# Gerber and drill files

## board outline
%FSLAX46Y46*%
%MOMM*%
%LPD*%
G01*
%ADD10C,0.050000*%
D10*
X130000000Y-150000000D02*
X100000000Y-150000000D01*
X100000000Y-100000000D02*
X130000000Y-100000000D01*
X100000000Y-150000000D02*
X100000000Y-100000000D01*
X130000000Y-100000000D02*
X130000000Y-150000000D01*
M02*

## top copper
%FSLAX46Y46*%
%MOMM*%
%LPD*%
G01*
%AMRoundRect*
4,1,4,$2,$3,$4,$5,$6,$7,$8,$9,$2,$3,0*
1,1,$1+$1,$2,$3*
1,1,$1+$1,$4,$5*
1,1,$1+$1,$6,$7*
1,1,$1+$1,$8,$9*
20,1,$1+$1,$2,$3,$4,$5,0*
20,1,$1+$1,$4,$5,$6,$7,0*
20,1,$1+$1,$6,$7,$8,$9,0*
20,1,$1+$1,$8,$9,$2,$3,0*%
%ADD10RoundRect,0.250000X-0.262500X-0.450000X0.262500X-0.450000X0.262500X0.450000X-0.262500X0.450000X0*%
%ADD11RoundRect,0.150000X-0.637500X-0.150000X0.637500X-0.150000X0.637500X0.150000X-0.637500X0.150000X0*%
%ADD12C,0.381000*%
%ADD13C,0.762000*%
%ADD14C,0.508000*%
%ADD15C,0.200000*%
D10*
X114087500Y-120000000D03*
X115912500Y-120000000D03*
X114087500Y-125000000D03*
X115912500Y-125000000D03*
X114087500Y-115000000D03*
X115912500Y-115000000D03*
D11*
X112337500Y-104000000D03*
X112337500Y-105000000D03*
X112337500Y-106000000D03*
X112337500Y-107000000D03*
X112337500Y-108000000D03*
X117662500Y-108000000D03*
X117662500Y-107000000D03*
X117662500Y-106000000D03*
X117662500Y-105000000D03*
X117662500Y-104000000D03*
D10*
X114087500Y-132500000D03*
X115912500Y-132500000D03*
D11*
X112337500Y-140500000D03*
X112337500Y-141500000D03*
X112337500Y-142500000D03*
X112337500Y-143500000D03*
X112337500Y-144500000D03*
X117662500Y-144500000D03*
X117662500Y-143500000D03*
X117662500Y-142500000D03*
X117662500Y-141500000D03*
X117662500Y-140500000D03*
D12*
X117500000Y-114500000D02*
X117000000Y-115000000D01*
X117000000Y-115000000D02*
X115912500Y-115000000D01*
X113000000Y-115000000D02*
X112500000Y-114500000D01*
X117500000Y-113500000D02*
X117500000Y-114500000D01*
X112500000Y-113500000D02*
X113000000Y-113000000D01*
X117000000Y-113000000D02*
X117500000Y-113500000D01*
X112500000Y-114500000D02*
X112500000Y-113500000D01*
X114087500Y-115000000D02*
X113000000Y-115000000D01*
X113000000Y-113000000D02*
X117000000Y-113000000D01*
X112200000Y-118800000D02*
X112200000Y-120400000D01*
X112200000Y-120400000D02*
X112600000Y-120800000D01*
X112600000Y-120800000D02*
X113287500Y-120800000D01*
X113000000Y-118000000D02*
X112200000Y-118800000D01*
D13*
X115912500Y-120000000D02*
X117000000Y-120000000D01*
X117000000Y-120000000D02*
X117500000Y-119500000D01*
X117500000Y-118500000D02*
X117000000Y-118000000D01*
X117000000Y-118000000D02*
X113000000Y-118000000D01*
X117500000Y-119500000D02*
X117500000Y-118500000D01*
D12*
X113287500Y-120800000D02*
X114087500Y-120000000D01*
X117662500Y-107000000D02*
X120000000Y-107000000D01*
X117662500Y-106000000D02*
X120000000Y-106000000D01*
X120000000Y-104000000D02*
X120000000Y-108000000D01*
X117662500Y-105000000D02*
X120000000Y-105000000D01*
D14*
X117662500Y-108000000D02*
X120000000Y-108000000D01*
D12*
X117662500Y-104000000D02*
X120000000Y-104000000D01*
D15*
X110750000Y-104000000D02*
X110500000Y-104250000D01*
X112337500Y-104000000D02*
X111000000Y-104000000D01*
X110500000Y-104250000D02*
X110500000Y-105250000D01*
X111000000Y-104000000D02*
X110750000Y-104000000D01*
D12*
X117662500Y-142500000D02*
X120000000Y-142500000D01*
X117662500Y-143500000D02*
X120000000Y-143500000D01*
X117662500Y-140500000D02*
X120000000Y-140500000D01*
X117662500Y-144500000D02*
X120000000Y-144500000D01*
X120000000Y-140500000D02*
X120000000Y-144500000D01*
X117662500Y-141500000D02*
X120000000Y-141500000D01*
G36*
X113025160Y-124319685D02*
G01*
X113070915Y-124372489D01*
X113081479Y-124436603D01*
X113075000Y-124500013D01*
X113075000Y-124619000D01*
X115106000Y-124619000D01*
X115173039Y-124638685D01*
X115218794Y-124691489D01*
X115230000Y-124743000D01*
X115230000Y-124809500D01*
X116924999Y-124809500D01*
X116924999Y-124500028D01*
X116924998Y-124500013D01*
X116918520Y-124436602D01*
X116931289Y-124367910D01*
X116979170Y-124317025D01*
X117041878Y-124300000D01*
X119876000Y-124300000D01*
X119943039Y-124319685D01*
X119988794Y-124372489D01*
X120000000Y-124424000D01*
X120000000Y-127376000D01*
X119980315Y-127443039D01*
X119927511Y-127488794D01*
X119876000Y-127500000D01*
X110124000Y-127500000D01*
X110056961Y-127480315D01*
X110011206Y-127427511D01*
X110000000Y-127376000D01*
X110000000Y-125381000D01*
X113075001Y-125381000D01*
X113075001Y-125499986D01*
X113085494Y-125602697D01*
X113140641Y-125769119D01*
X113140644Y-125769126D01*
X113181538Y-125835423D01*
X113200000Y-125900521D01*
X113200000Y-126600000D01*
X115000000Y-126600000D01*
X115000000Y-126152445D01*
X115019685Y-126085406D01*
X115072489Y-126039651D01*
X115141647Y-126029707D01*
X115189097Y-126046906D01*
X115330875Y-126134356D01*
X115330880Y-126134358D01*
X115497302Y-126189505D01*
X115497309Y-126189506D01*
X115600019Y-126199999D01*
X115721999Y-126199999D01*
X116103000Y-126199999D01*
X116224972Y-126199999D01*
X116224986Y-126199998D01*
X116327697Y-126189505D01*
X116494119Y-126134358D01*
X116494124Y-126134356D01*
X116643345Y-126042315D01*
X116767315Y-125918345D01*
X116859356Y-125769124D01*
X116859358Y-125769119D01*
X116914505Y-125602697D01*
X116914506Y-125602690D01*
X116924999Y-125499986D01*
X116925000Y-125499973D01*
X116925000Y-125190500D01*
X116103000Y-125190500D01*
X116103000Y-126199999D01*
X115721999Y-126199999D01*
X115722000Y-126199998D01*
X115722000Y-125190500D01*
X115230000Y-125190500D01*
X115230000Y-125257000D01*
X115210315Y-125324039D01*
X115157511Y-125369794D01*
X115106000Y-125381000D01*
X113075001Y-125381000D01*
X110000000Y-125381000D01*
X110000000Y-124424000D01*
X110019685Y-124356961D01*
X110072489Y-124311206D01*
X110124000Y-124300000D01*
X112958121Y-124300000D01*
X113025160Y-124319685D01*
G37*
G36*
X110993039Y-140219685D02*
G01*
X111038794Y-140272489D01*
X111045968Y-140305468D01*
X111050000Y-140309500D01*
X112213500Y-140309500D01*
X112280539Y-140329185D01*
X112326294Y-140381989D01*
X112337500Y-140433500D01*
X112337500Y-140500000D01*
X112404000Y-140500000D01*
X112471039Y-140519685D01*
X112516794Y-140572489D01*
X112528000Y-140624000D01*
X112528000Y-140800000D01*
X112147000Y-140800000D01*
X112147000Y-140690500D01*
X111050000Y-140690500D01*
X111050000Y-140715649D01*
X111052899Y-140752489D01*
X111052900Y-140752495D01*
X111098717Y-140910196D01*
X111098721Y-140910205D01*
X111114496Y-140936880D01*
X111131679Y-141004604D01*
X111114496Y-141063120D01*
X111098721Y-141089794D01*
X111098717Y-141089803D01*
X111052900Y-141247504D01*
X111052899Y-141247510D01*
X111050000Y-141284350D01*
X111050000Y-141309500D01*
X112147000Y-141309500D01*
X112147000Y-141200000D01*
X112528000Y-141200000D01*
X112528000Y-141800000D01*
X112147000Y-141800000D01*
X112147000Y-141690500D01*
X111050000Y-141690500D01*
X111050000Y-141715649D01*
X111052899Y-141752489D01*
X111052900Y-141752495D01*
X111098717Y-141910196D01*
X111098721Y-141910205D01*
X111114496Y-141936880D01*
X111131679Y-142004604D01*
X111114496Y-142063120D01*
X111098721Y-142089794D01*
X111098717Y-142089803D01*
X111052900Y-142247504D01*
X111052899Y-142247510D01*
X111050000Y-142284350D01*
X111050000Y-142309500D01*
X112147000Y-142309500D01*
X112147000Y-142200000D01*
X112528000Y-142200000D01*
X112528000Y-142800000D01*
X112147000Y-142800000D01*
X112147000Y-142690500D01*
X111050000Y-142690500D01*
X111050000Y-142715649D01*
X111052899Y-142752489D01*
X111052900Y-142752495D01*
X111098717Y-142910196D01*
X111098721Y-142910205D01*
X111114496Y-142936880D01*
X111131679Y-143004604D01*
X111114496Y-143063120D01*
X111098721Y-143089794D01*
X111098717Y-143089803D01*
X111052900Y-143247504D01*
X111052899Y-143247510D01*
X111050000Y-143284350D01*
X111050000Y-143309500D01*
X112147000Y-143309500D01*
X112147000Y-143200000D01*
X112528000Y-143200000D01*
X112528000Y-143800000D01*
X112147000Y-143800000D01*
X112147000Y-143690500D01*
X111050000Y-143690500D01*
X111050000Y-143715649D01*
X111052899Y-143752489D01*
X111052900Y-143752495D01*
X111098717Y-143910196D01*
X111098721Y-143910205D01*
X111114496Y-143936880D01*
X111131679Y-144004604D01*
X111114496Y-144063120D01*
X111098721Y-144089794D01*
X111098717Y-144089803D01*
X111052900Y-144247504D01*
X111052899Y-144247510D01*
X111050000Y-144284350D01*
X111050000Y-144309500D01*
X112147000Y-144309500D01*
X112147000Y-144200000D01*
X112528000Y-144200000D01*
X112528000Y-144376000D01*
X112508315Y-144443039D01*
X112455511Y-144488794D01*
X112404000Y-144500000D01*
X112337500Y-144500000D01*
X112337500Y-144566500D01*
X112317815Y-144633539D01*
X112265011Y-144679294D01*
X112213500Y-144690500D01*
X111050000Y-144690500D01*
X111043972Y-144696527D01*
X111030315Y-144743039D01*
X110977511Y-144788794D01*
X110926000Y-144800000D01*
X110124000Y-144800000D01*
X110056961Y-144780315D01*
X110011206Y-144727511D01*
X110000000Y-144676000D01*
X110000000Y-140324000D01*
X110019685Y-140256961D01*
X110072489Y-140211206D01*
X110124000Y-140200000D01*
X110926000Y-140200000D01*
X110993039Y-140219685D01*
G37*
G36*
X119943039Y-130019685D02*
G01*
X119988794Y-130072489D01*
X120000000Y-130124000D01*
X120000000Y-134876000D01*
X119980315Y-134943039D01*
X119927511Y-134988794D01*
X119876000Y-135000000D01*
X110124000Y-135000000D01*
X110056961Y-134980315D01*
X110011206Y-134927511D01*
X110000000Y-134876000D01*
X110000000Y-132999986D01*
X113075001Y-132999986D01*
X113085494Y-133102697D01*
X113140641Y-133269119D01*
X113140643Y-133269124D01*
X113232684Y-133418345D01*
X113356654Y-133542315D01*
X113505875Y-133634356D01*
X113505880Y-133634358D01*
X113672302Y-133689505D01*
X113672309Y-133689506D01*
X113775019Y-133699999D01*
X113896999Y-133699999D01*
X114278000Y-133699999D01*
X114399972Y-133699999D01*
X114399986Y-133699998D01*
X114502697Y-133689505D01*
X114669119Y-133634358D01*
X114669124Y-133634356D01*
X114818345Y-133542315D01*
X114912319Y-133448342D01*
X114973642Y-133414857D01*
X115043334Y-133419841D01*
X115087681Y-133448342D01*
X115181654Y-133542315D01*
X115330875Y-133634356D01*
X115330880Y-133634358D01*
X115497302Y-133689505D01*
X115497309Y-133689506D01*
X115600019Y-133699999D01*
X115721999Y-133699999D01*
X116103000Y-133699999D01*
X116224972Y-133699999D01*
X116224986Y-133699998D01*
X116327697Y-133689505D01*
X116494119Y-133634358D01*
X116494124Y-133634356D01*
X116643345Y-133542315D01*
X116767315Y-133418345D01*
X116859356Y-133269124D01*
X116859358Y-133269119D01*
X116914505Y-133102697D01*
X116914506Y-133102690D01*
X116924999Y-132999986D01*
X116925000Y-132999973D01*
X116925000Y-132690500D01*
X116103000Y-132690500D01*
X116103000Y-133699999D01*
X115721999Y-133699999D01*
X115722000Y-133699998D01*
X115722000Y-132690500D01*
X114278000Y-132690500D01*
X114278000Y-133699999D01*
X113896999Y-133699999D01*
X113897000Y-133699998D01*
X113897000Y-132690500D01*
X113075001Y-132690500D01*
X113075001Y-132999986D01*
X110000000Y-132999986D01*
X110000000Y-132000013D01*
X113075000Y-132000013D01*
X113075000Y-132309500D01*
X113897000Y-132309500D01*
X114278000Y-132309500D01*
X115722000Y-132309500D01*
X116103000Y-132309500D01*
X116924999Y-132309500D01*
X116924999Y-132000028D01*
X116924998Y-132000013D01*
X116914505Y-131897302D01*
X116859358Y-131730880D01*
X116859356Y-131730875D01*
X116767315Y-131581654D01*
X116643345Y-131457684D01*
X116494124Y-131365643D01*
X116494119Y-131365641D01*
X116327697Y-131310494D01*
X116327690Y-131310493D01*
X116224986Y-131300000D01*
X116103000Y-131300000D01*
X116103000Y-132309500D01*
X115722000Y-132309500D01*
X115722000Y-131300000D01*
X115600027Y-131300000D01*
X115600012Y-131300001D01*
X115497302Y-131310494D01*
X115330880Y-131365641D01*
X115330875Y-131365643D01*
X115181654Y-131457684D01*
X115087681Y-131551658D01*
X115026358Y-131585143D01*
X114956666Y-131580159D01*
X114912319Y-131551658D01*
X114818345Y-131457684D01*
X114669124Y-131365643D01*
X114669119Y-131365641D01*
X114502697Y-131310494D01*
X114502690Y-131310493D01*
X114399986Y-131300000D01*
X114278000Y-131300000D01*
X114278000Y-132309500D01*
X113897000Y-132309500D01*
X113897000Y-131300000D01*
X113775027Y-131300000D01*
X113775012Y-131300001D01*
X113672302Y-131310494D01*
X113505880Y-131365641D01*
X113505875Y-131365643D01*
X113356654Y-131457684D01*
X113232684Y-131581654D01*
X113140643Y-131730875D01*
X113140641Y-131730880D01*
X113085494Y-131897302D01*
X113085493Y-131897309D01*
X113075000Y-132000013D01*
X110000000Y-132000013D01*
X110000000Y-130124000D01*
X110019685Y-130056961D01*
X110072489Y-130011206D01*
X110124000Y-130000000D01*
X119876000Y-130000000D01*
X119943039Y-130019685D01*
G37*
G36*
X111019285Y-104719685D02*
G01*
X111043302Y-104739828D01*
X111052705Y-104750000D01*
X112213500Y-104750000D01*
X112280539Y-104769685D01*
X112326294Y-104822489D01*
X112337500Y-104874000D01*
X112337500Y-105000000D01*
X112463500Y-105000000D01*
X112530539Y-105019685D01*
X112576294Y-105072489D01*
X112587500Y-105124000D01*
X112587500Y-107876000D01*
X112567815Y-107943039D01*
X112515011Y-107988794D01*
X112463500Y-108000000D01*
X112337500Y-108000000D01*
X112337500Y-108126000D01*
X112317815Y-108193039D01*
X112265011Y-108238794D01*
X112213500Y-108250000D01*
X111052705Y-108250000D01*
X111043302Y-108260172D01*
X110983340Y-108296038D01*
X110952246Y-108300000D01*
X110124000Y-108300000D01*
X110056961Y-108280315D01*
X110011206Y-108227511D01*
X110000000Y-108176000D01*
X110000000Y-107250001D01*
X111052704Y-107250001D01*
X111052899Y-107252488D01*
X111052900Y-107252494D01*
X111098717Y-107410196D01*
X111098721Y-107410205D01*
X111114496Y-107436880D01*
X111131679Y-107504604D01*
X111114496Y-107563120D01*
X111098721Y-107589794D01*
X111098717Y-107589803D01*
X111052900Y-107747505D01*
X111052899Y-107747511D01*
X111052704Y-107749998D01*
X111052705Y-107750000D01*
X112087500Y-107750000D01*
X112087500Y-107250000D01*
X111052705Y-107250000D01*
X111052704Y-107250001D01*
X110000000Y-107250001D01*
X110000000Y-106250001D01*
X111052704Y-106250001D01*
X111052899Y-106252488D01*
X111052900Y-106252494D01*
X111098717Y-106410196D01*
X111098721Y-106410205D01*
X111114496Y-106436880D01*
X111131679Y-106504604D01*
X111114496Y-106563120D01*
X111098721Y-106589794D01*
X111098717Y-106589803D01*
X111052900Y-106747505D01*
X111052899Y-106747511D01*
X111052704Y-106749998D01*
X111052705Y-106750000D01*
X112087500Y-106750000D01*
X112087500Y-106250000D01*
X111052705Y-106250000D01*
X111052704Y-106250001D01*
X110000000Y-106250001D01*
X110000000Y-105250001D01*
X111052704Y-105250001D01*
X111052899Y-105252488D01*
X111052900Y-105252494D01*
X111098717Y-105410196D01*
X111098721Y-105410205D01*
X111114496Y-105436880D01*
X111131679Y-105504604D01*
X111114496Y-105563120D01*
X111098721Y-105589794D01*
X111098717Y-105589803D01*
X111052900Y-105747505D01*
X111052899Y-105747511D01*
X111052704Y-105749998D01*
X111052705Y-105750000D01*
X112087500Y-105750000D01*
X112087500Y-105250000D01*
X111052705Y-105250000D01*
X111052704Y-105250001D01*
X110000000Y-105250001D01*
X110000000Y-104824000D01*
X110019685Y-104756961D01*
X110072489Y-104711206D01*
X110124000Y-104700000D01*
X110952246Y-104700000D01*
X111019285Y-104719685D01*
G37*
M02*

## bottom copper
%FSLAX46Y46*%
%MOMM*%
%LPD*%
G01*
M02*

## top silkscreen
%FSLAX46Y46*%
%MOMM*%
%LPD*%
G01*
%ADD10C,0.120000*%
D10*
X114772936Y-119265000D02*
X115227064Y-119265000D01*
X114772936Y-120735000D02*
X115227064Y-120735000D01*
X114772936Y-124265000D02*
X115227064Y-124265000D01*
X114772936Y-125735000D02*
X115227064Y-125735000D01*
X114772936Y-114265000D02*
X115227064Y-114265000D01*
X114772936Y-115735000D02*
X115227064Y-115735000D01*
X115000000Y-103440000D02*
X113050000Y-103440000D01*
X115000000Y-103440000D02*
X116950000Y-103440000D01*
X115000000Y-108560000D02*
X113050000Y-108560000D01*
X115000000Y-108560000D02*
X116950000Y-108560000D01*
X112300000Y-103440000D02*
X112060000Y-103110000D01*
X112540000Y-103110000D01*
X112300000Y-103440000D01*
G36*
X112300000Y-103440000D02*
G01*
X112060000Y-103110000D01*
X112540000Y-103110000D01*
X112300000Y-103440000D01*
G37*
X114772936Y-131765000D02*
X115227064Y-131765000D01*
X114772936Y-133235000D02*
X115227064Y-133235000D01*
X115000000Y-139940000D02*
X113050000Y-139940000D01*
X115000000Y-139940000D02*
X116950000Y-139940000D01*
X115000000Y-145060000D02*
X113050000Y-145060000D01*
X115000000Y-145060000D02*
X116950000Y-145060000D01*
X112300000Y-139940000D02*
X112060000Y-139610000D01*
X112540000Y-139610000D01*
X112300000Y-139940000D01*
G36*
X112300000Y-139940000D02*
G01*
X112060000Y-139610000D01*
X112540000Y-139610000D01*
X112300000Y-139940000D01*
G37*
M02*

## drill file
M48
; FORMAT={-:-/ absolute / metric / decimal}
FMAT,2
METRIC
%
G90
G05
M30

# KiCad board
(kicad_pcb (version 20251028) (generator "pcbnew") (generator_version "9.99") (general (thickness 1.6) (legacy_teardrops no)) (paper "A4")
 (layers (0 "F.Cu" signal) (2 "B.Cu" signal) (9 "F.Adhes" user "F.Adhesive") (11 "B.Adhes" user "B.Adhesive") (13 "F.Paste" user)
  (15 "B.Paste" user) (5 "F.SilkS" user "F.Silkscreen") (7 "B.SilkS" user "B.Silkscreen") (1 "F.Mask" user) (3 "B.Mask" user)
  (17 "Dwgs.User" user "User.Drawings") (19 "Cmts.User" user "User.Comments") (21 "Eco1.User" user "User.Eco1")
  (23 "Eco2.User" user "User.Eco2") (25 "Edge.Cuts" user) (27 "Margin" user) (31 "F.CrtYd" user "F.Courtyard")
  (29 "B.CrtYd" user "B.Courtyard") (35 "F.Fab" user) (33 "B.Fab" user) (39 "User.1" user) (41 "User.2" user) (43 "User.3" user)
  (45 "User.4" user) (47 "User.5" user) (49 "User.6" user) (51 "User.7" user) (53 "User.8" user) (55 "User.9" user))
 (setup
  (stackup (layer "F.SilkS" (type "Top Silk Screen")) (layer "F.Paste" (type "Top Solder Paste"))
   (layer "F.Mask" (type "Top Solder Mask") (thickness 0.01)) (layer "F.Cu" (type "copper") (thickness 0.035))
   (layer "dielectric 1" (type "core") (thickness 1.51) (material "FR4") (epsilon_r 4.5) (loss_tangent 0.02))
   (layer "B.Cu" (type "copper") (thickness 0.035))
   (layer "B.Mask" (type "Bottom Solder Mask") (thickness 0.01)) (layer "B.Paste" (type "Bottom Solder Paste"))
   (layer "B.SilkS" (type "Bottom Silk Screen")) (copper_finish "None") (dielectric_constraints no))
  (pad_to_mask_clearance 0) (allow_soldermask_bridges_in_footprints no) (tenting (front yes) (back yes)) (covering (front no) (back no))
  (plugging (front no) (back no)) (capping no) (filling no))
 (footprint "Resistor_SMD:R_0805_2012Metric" (layer "F.Cu") (at 115 120)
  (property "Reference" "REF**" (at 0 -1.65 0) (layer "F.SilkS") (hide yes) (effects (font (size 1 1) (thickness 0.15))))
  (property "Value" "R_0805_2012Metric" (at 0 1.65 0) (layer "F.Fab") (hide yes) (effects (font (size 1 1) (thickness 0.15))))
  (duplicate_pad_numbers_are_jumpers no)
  (fp_line (start -0.227064 -0.735) (end 0.227064 -0.735) (stroke (width 0.12) (type solid)) (layer "F.SilkS"))
  (fp_line (start -0.227064 0.735) (end 0.227064 0.735) (stroke (width 0.12) (type solid)) (layer "F.SilkS"))
  (pad "1" smd roundrect (at -0.9125 0) (size 1.025 1.4) (layers "F.Cu" "F.Mask" "F.Paste") (roundrect_rratio 0.243902) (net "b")
   (tenting (front none) (back none)))
  (pad "2" smd roundrect (at 0.9125 0) (size 1.025 1.4) (layers "F.Cu" "F.Mask" "F.Paste") (roundrect_rratio 0.243902) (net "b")
   (tenting (front none) (back none))))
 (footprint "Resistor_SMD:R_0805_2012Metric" (layer "F.Cu") (at 115 125)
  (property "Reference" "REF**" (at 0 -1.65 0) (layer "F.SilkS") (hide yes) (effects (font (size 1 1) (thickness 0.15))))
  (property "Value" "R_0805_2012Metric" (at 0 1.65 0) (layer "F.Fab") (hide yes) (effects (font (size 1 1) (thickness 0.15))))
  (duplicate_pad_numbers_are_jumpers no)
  (fp_line (start -0.227064 -0.735) (end 0.227064 -0.735) (stroke (width 0.12) (type solid)) (layer "F.SilkS"))
  (fp_line (start -0.227064 0.735) (end 0.227064 0.735) (stroke (width 0.12) (type solid)) (layer "F.SilkS"))
  (pad "1" smd roundrect (at -0.9125 0) (size 1.025 1.4) (layers "F.Cu" "F.Mask" "F.Paste") (roundrect_rratio 0.243902) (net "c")
   (tenting (front none) (back none)))
  (pad "2" smd roundrect (at 0.9125 0) (size 1.025 1.4) (layers "F.Cu" "F.Mask" "F.Paste") (roundrect_rratio 0.243902) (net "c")
   (thermal_bridge_width 0.381) (tenting (front none) (back none))))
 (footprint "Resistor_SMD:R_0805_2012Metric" (layer "F.Cu") (at 115 115)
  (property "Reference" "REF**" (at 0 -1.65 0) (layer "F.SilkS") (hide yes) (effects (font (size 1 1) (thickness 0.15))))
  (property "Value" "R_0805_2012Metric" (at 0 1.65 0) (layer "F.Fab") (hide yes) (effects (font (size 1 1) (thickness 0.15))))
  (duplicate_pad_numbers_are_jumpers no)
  (fp_line (start -0.227064 -0.735) (end 0.227064 -0.735) (stroke (width 0.12) (type solid)) (layer "F.SilkS"))
  (fp_line (start -0.227064 0.735) (end 0.227064 0.735) (stroke (width 0.12) (type solid)) (layer "F.SilkS"))
  (pad "1" smd roundrect (at -0.9125 0) (size 1.025 1.4) (layers "F.Cu" "F.Mask" "F.Paste") (roundrect_rratio 0.243902) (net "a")
   (tenting (front none) (back none)))
  (pad "2" smd roundrect (at 0.9125 0) (size 1.025 1.4) (layers "F.Cu" "F.Mask" "F.Paste") (roundrect_rratio 0.243902) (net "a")
   (tenting (front none) (back none))))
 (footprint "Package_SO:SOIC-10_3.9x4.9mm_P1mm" (layer "F.Cu") (at 115 106)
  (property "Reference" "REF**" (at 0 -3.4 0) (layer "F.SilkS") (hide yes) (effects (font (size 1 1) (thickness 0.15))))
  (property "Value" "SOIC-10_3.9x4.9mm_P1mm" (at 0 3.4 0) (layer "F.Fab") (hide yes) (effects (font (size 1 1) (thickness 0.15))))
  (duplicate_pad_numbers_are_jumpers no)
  (fp_line (start 0 -2.56) (end -1.95 -2.56) (stroke (width 0.12) (type solid)) (layer "F.SilkS"))
  (fp_line (start 0 -2.56) (end 1.95 -2.56) (stroke (width 0.12) (type solid)) (layer "F.SilkS"))
  (fp_line (start 0 2.56) (end -1.95 2.56) (stroke (width 0.12) (type solid)) (layer "F.SilkS"))
  (fp_line (start 0 2.56) (end 1.95 2.56) (stroke (width 0.12) (type solid)) (layer "F.SilkS"))
  (fp_poly
   (pts (xy -2.7 -2.56) (xy -2.94 -2.89) (xy -2.46 -2.89) (xy -2.7 -2.56)) (stroke (width 0.12) (type solid)) (fill yes) (layer "F.SilkS"))
  (pad "1" smd roundrect (at -2.6625 -2) (size 1.575 0.6) (layers "F.Cu" "F.Mask" "F.Paste") (roundrect_rratio 0.25) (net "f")
   (tenting (front none) (back none)))
  (pad "2" smd roundrect (at -2.6625 -1) (size 1.575 0.6) (layers "F.Cu" "F.Mask" "F.Paste") (roundrect_rratio 0.25) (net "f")
   (tenting (front none) (back none)))
  (pad "3" smd roundrect (at -2.6625 0) (size 1.575 0.6) (layers "F.Cu" "F.Mask" "F.Paste") (roundrect_rratio 0.25) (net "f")
   (tenting (front none) (back none)))
  (pad "4" smd roundrect (at -2.6625 1) (size 1.575 0.6) (layers "F.Cu" "F.Mask" "F.Paste") (roundrect_rratio 0.25) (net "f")
   (tenting (front none) (back none)))
  (pad "5" smd roundrect (at -2.6625 2) (size 1.575 0.6) (layers "F.Cu" "F.Mask" "F.Paste") (roundrect_rratio 0.25) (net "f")
   (tenting (front none) (back none)))
  (pad "6" smd roundrect (at 2.6625 2) (size 1.575 0.6) (layers "F.Cu" "F.Mask" "F.Paste") (roundrect_rratio 0.25) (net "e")
   (tenting (front none) (back none)))
  (pad "7" smd roundrect (at 2.6625 1) (size 1.575 0.6) (layers "F.Cu" "F.Mask" "F.Paste") (roundrect_rratio 0.25) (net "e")
   (tenting (front none) (back none)))
  (pad "8" smd roundrect (at 2.6625 0) (size 1.575 0.6) (layers "F.Cu" "F.Mask" "F.Paste") (roundrect_rratio 0.25) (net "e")
   (tenting (front none) (back none)))
  (pad "9" smd roundrect (at 2.6625 -1) (size 1.575 0.6) (layers "F.Cu" "F.Mask" "F.Paste") (roundrect_rratio 0.25) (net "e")
   (tenting (front none) (back none)))
  (pad "10" smd roundrect (at 2.6625 -2) (size 1.575 0.6) (layers "F.Cu" "F.Mask" "F.Paste") (roundrect_rratio 0.25) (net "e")
   (tenting (front none) (back none))))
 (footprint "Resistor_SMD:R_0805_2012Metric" (layer "F.Cu") (at 115 132.5)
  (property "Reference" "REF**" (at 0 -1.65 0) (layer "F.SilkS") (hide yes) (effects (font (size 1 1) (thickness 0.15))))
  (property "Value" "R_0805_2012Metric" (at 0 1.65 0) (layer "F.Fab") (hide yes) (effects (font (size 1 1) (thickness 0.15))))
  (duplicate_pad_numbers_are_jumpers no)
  (fp_line (start -0.227064 -0.735) (end 0.227064 -0.735) (stroke (width 0.12) (type solid)) (layer "F.SilkS"))
  (fp_line (start -0.227064 0.735) (end 0.227064 0.735) (stroke (width 0.12) (type solid)) (layer "F.SilkS"))
  (pad "1" smd roundrect (at -0.9125 0) (size 1.025 1.4) (layers "F.Cu" "F.Mask" "F.Paste") (roundrect_rratio 0.243902) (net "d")
   (tenting (front none) (back none)))
  (pad "2" smd roundrect (at 0.9125 0) (size 1.025 1.4) (layers "F.Cu" "F.Mask" "F.Paste") (roundrect_rratio 0.243902) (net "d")
   (tenting (front none) (back none))))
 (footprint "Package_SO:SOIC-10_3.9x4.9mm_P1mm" (layer "F.Cu") (at 115 142.5)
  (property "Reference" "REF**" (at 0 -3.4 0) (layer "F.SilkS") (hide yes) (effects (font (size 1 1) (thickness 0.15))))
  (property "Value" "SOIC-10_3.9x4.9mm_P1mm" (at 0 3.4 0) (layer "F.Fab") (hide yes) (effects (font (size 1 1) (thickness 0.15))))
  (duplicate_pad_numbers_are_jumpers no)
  (fp_line (start 0 -2.56) (end -1.95 -2.56) (stroke (width 0.12) (type solid)) (layer "F.SilkS"))
  (fp_line (start 0 -2.56) (end 1.95 -2.56) (stroke (width 0.12) (type solid)) (layer "F.SilkS"))
  (fp_line (start 0 2.56) (end -1.95 2.56) (stroke (width 0.12) (type solid)) (layer "F.SilkS"))
  (fp_line (start 0 2.56) (end 1.95 2.56) (stroke (width 0.12) (type solid)) (layer "F.SilkS"))
  (fp_poly
   (pts (xy -2.7 -2.56) (xy -2.94 -2.89) (xy -2.46 -2.89) (xy -2.7 -2.56)) (stroke (width 0.12) (type solid)) (fill yes) (layer "F.SilkS"))
  (pad "1" smd roundrect (at -2.6625 -2) (size 1.575 0.6) (layers "F.Cu" "F.Mask" "F.Paste") (roundrect_rratio 0.25) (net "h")
   (tenting (front none) (back none)))
  (pad "2" smd roundrect (at -2.6625 -1) (size 1.575 0.6) (layers "F.Cu" "F.Mask" "F.Paste") (roundrect_rratio 0.25) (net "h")
   (tenting (front none) (back none)))
  (pad "3" smd roundrect (at -2.6625 0) (size 1.575 0.6) (layers "F.Cu" "F.Mask" "F.Paste") (roundrect_rratio 0.25) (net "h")
   (tenting (front none) (back none)))
  (pad "4" smd roundrect (at -2.6625 1) (size 1.575 0.6) (layers "F.Cu" "F.Mask" "F.Paste") (roundrect_rratio 0.25) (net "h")
   (tenting (front none) (back none)))
  (pad "5" smd roundrect (at -2.6625 2) (size 1.575 0.6) (layers "F.Cu" "F.Mask" "F.Paste") (roundrect_rratio 0.25) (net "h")
   (tenting (front none) (back none)))
  (pad "6" smd roundrect (at 2.6625 2) (size 1.575 0.6) (layers "F.Cu" "F.Mask" "F.Paste") (roundrect_rratio 0.25) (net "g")
   (tenting (front none) (back none)))
  (pad "7" smd roundrect (at 2.6625 1) (size 1.575 0.6) (layers "F.Cu" "F.Mask" "F.Paste") (roundrect_rratio 0.25) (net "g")
   (tenting (front none) (back none)))
  (pad "8" smd roundrect (at 2.6625 0) (size 1.575 0.6) (layers "F.Cu" "F.Mask" "F.Paste") (roundrect_rratio 0.25) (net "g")
   (tenting (front none) (back none)))
  (pad "9" smd roundrect (at 2.6625 -1) (size 1.575 0.6) (layers "F.Cu" "F.Mask" "F.Paste") (roundrect_rratio 0.25) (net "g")
   (tenting (front none) (back none)))
  (pad "10" smd roundrect (at 2.6625 -2) (size 1.575 0.6) (layers "F.Cu" "F.Mask" "F.Paste") (roundrect_rratio 0.25) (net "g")
   (tenting (front none) (back none))))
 (gr_line (start 130 150) (end 100 150) (stroke (width 0.05) (type default)) (layer "Edge.Cuts"))
 (gr_line (start 100 100) (end 130 100) (stroke (width 0.05) (type default)) (layer "Edge.Cuts"))
 (gr_line (start 100 150) (end 100 100) (stroke (width 0.05) (type default)) (layer "Edge.Cuts"))
 (gr_line (start 130 100) (end 130 150) (stroke (width 0.05) (type default)) (layer "Edge.Cuts"))
 (segment (start 117.5 114.5) (end 117 115) (width 0.381) (layer "F.Cu") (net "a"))
 (segment (start 117 115) (end 115.9125 115) (width 0.381) (layer "F.Cu") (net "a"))
 (segment (start 113 115) (end 112.5 114.5) (width 0.381) (layer "F.Cu") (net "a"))
 (segment (start 117.5 113.5) (end 117.5 114.5) (width 0.381) (layer "F.Cu") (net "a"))
 (segment (start 112.5 113.5) (end 113 113) (width 0.381) (layer "F.Cu") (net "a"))
 (segment (start 117 113) (end 117.5 113.5) (width 0.381) (layer "F.Cu") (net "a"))
 (segment (start 112.5 114.5) (end 112.5 113.5) (width 0.381) (layer "F.Cu") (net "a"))
 (segment (start 114.0875 115) (end 113 115) (width 0.381) (layer "F.Cu") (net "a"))
 (segment (start 113 113) (end 117 113) (width 0.381) (layer "F.Cu") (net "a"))
 (segment (start 112.2 118.8) (end 112.2 120.4) (width 0.381) (layer "F.Cu") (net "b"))
 (segment (start 112.2 120.4) (end 112.6 120.8) (width 0.381) (layer "F.Cu") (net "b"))
 (segment (start 112.6 120.8) (end 113.2875 120.8) (width 0.381) (layer "F.Cu") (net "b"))
 (segment (start 113 118) (end 112.2 118.8) (width 0.381) (layer "F.Cu") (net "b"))
 (segment (start 115.9125 120) (end 117 120) (width 0.762) (layer "F.Cu") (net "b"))
 (segment (start 117 120) (end 117.5 119.5) (width 0.762) (layer "F.Cu") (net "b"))
 (segment (start 117.5 118.5) (end 117 118) (width 0.762) (layer "F.Cu") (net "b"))
 (segment (start 117 118) (end 113 118) (width 0.762) (layer "F.Cu") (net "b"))
 (segment (start 117.5 119.5) (end 117.5 118.5) (width 0.762) (layer "F.Cu") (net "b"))
 (segment (start 113.2875 120.8) (end 114.0875 120) (width 0.381) (layer "F.Cu") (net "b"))
 (segment (start 117.6625 107) (end 120 107) (width 0.381) (layer "F.Cu") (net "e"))
 (segment (start 117.6625 106) (end 120 106) (width 0.381) (layer "F.Cu") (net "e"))
 (segment (start 120 104) (end 120 108) (width 0.381) (layer "F.Cu") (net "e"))
 (segment (start 117.6625 105) (end 120 105) (width 0.381) (layer "F.Cu") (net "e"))
 (segment (start 117.6625 108) (end 120 108) (width 0.508) (layer "F.Cu") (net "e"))
 (segment (start 117.6625 104) (end 120 104) (width 0.381) (layer "F.Cu") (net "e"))
 (segment (start 110.75 104) (end 110.5 104.25) (width 0.2) (layer "F.Cu") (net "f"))
 (segment (start 112.3375 104) (end 111 104) (width 0.2) (layer "F.Cu") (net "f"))
 (segment (start 110.5 104.25) (end 110.5 105.25) (width 0.2) (layer "F.Cu") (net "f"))
 (segment (start 111 104) (end 110.75 104) (width 0.2) (layer "F.Cu") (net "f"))
 (segment (start 117.6625 142.5) (end 120 142.5) (width 0.381) (layer "F.Cu") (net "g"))
 (segment (start 117.6625 143.5) (end 120 143.5) (width 0.381) (layer "F.Cu") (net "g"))
 (segment (start 117.6625 140.5) (end 120 140.5) (width 0.381) (layer "F.Cu") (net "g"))
 (segment (start 117.6625 144.5) (end 120 144.5) (width 0.381) (layer "F.Cu") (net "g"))
 (segment (start 120 140.5) (end 120 144.5) (width 0.381) (layer "F.Cu") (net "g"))
 (segment (start 117.6625 141.5) (end 120 141.5) (width 0.381) (layer "F.Cu") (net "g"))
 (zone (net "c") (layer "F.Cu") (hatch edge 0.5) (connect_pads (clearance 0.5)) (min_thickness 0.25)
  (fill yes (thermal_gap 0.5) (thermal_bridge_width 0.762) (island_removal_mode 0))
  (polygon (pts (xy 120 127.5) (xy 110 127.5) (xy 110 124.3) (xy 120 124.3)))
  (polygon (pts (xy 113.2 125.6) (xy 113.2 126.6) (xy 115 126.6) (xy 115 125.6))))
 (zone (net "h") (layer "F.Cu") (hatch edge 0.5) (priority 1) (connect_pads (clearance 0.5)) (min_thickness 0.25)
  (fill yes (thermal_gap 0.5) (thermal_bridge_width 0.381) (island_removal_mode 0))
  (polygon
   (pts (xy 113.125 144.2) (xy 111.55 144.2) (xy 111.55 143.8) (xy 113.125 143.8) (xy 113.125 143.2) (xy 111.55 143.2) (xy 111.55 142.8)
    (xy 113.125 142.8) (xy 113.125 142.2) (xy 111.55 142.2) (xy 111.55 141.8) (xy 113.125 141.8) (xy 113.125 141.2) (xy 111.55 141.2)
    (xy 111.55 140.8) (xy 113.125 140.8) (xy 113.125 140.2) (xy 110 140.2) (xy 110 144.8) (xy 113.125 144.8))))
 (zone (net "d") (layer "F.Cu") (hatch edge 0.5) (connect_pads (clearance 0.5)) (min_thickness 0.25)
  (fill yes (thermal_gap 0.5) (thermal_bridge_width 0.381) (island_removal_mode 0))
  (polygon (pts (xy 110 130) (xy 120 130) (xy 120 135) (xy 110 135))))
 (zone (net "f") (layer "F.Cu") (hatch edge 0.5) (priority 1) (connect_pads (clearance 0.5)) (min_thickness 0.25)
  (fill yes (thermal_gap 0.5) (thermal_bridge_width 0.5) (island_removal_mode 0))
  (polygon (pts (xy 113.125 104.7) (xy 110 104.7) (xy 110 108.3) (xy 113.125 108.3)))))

